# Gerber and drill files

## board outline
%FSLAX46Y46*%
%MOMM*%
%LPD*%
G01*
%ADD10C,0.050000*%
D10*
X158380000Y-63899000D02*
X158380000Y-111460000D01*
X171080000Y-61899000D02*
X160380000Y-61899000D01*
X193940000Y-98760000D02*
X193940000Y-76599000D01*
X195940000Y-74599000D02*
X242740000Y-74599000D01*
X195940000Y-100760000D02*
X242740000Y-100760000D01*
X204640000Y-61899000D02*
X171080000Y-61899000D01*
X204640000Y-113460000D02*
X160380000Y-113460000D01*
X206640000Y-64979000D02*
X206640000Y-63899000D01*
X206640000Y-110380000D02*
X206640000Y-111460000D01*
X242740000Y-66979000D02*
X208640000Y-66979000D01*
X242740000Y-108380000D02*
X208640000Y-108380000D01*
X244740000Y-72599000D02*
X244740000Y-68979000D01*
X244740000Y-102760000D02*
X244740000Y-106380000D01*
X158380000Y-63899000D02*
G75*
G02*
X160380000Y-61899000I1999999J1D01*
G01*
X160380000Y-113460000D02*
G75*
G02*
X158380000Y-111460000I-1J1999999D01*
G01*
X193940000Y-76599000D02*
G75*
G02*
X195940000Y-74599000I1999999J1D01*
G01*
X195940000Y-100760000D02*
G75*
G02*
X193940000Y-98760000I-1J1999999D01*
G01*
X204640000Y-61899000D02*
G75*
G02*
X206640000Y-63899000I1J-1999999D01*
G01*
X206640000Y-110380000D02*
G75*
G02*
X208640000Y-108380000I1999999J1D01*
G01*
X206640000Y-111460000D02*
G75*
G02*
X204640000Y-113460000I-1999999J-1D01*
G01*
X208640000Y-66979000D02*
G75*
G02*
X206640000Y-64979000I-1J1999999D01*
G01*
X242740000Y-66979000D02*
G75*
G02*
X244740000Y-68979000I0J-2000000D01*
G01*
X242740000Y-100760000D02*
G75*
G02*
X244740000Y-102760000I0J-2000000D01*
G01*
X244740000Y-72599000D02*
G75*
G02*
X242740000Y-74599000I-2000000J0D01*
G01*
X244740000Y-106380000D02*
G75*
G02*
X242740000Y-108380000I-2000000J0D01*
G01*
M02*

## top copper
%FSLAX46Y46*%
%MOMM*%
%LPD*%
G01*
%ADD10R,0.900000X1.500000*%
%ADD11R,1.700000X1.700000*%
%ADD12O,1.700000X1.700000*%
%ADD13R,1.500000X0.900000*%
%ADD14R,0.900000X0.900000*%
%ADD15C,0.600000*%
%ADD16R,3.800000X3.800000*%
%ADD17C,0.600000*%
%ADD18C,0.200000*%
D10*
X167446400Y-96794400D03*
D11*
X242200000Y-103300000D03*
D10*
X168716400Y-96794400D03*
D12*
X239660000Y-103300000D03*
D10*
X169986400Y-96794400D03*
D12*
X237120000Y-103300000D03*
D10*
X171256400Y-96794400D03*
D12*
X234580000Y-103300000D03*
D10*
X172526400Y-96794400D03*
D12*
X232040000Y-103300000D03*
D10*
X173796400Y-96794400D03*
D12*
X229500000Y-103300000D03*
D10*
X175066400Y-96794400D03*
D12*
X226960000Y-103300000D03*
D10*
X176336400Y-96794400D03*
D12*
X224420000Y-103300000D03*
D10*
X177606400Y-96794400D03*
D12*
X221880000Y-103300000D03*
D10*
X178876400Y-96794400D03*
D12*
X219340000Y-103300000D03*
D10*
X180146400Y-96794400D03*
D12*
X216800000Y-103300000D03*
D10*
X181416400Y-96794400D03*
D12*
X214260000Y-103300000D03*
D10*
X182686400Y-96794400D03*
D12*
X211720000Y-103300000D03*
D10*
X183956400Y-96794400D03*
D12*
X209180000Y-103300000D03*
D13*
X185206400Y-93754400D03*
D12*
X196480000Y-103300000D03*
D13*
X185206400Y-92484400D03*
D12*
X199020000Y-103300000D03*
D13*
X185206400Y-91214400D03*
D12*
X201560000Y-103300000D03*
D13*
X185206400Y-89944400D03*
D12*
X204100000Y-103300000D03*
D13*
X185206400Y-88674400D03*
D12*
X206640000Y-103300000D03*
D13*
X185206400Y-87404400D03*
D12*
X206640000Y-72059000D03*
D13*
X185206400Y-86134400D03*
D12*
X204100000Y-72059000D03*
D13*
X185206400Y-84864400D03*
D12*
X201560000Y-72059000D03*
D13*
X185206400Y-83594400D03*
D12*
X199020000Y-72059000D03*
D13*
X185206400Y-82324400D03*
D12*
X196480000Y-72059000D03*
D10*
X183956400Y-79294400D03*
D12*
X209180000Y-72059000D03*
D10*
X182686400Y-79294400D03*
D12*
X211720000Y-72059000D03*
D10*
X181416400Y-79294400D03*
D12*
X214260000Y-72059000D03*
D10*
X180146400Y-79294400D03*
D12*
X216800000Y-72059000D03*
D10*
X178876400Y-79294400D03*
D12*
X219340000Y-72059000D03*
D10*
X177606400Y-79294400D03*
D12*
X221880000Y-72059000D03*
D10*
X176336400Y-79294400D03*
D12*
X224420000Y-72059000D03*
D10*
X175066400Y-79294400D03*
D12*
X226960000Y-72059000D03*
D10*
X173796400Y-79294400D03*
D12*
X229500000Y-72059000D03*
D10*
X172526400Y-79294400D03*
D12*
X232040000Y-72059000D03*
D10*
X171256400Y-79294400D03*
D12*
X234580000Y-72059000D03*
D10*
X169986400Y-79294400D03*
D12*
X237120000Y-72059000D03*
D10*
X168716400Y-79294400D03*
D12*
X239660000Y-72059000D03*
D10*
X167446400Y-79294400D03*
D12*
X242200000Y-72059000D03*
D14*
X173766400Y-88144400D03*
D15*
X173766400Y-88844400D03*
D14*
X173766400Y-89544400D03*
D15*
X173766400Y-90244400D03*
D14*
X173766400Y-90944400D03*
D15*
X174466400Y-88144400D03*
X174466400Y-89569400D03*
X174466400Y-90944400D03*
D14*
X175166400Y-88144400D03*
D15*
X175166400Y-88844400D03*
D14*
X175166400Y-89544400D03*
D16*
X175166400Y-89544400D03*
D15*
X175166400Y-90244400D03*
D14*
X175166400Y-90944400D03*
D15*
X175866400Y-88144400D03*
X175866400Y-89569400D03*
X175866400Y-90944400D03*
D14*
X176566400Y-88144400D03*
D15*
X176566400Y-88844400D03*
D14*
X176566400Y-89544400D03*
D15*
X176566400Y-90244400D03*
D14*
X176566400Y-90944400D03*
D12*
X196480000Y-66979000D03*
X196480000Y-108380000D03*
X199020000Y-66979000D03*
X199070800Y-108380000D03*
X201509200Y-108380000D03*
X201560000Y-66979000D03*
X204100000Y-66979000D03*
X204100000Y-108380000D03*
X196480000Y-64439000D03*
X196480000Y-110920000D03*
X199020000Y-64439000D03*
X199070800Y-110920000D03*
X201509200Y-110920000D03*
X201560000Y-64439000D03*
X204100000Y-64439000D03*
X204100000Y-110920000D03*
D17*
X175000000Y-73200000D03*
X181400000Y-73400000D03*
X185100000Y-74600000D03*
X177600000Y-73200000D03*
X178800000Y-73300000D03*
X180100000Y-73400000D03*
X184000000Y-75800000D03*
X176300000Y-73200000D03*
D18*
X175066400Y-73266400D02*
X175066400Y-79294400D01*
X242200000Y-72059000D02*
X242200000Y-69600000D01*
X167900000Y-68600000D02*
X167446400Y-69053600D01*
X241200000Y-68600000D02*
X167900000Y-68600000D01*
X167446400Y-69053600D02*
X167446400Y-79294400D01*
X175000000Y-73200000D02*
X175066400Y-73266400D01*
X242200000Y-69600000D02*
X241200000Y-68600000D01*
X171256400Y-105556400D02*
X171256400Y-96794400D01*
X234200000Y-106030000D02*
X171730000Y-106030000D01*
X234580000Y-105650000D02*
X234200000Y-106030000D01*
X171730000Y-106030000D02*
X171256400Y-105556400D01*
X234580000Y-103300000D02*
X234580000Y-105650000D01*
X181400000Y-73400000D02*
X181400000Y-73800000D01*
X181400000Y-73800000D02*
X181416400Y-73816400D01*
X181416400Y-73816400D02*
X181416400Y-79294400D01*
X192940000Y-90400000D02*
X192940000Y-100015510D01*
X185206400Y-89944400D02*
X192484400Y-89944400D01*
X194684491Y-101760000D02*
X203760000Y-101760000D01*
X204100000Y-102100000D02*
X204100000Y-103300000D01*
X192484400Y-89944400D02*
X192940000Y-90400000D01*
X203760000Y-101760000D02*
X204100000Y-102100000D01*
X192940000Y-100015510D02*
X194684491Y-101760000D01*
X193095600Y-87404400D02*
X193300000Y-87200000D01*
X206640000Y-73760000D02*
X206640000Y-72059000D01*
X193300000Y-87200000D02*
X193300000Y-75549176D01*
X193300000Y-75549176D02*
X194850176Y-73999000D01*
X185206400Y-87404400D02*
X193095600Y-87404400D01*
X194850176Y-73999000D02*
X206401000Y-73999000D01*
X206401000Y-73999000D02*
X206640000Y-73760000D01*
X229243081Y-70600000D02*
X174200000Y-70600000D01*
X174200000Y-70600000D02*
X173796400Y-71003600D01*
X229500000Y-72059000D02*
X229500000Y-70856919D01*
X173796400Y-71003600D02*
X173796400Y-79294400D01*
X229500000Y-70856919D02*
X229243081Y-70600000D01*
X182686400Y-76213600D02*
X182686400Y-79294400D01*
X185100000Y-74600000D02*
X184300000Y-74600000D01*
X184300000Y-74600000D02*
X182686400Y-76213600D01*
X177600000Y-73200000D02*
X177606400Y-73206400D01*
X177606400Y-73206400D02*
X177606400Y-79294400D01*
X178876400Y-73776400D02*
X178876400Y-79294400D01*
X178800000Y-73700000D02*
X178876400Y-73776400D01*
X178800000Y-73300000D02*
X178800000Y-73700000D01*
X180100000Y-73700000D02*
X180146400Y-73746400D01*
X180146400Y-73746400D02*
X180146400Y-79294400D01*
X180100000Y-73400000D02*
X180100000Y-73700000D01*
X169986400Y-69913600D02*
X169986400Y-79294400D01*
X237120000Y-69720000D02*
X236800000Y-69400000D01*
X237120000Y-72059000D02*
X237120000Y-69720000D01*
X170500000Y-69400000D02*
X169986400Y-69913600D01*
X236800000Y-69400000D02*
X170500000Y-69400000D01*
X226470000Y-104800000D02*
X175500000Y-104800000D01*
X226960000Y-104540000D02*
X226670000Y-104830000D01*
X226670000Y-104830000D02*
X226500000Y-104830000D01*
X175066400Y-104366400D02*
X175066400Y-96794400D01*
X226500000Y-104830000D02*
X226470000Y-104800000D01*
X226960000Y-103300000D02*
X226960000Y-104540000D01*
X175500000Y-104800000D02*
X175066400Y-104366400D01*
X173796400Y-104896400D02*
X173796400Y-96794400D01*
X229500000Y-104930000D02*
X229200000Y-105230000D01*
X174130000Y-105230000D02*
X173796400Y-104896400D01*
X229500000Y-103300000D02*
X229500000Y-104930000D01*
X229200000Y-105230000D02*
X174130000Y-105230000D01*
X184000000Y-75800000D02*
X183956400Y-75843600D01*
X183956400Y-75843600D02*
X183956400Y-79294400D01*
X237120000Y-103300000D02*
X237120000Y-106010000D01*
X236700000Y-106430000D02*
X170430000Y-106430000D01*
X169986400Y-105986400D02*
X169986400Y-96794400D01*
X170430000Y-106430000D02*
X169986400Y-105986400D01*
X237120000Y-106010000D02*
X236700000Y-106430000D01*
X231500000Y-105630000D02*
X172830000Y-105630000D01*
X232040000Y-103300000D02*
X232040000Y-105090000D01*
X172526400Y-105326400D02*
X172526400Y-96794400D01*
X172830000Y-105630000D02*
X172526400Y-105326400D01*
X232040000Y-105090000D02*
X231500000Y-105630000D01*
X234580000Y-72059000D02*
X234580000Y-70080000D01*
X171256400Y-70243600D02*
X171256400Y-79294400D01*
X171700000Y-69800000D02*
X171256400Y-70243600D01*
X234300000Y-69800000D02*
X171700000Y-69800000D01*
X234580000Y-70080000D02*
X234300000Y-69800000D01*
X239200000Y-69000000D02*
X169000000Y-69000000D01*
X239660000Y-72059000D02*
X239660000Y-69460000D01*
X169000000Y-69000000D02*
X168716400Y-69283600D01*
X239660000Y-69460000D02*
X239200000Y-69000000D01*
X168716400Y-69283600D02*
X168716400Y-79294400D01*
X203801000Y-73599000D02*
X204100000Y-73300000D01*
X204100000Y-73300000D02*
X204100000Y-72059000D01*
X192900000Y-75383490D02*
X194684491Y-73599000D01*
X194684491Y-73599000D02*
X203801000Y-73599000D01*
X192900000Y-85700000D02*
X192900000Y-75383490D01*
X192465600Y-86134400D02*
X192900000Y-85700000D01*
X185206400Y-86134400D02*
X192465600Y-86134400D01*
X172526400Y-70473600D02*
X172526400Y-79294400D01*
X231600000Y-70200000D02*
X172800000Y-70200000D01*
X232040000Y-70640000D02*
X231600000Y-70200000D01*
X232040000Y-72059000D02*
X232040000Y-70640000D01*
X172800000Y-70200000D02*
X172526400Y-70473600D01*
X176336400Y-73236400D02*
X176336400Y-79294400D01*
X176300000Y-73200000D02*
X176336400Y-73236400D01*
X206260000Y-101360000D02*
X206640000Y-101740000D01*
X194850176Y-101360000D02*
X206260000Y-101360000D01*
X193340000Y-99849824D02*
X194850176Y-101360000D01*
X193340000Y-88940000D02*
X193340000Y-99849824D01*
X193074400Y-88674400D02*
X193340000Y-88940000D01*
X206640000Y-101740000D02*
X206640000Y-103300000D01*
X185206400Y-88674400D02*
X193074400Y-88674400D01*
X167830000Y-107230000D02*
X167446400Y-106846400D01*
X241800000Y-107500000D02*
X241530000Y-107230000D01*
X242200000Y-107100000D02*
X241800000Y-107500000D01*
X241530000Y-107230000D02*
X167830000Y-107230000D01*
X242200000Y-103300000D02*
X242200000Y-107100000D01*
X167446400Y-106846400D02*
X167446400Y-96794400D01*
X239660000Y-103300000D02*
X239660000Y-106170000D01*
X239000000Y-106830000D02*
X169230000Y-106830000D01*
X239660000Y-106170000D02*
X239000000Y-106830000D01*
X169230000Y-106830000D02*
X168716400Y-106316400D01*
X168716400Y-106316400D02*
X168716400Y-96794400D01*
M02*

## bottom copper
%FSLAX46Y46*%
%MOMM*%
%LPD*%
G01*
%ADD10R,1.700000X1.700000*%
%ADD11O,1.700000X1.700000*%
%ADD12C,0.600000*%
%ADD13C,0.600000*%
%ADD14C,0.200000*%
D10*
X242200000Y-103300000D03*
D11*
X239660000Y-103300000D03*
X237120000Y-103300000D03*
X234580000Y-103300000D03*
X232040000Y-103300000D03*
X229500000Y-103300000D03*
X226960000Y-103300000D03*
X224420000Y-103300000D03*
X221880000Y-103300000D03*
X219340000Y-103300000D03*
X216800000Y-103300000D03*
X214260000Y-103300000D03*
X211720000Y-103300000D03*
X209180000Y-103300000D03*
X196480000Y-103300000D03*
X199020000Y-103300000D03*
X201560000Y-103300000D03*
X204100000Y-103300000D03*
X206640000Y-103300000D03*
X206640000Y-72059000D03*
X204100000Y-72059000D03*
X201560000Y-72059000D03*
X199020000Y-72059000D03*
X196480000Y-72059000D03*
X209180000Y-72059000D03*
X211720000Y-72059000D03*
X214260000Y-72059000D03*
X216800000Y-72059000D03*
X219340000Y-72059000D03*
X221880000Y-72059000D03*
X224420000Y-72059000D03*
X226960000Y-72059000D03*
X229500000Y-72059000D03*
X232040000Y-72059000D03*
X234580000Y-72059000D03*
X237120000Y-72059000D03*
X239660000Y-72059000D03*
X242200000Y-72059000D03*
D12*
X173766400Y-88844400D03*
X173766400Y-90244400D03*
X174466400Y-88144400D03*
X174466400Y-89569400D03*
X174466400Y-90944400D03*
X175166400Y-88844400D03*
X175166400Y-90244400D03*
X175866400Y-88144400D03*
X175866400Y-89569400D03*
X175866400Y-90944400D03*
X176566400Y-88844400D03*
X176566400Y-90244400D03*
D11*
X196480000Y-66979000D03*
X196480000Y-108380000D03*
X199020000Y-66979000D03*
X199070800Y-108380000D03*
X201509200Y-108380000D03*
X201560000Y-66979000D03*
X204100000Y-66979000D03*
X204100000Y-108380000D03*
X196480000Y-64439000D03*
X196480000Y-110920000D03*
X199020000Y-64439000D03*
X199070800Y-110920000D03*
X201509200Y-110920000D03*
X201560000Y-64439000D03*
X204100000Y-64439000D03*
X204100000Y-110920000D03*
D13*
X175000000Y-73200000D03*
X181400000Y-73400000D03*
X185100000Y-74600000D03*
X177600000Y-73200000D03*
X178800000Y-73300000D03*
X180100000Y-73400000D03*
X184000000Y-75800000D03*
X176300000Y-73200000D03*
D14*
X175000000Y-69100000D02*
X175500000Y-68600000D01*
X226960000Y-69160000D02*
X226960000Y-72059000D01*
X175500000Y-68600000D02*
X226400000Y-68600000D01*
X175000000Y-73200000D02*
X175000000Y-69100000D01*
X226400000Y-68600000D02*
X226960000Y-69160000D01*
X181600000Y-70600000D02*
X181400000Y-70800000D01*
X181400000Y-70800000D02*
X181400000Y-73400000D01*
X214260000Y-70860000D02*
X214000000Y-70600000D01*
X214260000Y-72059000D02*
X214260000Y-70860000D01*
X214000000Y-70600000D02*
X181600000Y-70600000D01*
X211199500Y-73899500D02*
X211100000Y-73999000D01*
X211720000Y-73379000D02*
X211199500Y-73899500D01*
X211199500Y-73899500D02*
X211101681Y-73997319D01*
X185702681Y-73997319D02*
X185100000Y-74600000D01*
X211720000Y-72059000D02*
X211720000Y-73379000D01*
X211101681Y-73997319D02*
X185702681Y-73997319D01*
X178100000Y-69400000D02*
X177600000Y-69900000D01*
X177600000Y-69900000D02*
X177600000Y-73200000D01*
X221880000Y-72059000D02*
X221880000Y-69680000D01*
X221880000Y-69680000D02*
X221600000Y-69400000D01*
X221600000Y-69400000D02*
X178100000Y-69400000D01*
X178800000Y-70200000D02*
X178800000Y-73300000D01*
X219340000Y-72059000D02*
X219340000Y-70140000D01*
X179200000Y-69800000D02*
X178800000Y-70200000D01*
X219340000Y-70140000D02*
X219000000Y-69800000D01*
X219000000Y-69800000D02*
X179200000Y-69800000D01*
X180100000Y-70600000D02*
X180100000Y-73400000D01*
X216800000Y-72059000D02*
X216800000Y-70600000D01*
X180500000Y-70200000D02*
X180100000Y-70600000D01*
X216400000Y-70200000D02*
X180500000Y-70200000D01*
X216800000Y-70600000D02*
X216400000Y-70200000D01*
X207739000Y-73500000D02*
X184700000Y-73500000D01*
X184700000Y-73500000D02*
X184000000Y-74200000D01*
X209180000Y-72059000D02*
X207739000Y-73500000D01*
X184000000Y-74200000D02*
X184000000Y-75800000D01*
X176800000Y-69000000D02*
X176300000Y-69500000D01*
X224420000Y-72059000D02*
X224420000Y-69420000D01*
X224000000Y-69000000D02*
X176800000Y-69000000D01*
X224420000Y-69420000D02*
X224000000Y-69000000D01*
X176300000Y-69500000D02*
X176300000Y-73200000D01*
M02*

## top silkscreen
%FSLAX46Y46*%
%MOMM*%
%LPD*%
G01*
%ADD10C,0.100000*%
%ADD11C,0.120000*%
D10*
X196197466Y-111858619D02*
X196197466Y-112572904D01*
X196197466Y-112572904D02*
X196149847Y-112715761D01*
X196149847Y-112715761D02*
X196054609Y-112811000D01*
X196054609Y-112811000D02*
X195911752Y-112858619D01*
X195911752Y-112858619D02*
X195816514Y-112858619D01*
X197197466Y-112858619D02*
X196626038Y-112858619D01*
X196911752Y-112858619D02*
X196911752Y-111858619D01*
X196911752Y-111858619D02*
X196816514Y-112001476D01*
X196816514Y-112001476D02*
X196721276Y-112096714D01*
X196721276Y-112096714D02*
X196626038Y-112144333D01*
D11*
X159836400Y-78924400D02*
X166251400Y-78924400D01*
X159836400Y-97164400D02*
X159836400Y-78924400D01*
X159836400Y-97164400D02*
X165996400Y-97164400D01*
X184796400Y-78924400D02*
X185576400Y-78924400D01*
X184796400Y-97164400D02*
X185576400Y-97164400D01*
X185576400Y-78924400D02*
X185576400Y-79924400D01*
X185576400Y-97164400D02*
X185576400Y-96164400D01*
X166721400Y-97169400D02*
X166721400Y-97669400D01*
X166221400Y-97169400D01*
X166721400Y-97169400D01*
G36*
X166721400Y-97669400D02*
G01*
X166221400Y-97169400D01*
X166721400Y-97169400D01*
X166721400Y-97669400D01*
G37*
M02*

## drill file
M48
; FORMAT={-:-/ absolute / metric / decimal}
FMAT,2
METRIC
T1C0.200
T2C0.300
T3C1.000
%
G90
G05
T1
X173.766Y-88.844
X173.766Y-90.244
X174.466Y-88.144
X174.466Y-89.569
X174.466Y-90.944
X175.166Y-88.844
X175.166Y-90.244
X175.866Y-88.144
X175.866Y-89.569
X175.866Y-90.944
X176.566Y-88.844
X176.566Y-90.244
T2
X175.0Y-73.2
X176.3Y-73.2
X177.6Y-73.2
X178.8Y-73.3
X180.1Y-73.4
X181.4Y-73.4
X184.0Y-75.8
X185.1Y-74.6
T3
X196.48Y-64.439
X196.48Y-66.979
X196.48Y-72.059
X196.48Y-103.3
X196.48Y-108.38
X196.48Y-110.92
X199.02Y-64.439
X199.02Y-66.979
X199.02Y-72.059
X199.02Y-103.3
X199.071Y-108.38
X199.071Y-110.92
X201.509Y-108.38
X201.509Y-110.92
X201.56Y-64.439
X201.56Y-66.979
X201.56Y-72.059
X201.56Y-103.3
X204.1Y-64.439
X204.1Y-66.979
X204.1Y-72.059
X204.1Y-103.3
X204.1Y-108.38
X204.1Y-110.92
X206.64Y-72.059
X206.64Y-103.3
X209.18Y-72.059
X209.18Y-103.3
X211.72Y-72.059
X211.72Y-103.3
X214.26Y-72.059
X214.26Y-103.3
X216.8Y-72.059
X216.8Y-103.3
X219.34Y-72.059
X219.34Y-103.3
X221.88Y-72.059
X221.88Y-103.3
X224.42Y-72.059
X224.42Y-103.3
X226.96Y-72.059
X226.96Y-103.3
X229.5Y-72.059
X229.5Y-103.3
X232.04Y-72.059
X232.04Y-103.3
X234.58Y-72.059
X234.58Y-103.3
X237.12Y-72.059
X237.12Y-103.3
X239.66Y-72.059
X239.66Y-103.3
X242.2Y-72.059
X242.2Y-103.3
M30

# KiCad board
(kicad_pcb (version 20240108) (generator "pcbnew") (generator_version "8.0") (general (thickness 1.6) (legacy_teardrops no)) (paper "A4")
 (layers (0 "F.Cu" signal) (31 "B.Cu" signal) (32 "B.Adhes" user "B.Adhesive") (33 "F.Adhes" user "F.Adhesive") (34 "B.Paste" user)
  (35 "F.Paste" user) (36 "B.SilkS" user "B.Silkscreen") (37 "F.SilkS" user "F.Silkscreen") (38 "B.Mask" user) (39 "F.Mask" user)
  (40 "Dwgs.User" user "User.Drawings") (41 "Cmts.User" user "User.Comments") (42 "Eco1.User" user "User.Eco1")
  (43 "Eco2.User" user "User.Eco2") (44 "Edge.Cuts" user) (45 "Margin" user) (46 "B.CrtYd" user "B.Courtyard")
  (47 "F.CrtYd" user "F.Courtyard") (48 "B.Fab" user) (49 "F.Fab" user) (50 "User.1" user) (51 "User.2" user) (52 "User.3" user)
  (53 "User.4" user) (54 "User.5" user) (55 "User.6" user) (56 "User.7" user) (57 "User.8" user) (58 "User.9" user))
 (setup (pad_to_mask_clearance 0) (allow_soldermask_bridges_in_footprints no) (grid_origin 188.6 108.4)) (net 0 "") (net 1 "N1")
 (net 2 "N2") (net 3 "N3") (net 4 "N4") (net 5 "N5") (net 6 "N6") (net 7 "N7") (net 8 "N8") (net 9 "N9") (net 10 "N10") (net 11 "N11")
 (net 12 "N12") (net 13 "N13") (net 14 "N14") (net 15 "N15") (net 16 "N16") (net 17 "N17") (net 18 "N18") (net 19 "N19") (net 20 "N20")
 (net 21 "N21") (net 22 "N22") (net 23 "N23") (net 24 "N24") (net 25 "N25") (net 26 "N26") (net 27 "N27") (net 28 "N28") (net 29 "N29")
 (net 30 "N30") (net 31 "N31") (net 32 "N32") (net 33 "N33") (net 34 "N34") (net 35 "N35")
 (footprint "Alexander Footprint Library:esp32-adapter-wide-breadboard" (layer "F.Cu") (at 211.72 108.38)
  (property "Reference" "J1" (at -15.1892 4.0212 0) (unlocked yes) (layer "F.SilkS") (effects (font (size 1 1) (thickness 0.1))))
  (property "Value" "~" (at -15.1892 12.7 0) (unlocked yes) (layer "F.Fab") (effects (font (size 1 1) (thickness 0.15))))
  (fp_line (start -51.8836 -29.4556) (end -45.4686 -29.4556) (stroke (width 0.12) (type solid)) (layer "F.SilkS"))
  (fp_line (start -51.8836 -11.2156) (end -51.8836 -29.4556) (stroke (width 0.12) (type solid)) (layer "F.SilkS"))
  (fp_line (start -51.8836 -11.2156) (end -45.7236 -11.2156) (stroke (width 0.12) (type solid)) (layer "F.SilkS"))
  (fp_line (start -26.9236 -29.4556) (end -26.1436 -29.4556) (stroke (width 0.12) (type solid)) (layer "F.SilkS"))
  (fp_line (start -26.9236 -11.2156) (end -26.1436 -11.2156) (stroke (width 0.12) (type solid)) (layer "F.SilkS"))
  (fp_line (start -26.1436 -29.4556) (end -26.1436 -28.4556) (stroke (width 0.12) (type solid)) (layer "F.SilkS"))
  (fp_line (start -26.1436 -11.2156) (end -26.1436 -12.2156) (stroke (width 0.12) (type solid)) (layer "F.SilkS"))
  (fp_poly
   (pts (xy -44.9986 -11.2106) (xy -44.9986 -10.7106) (xy -45.4986 -11.2106) (xy -44.9986 -11.2106)) (stroke (width 0.12) (type solid))
   (fill solid) (layer "F.SilkS"))
  (fp_line (start -53.34 -44.481) (end -53.34 3.08) (stroke (width 0.05) (type default)) (layer "Edge.Cuts"))
  (fp_line (start -40.64 -46.481) (end -51.34 -46.481) (stroke (width 0.05) (type default)) (layer "Edge.Cuts"))
  (fp_line (start -17.78 -9.62) (end -17.78 -31.781) (stroke (width 0.05) (type default)) (layer "Edge.Cuts"))
  (fp_line (start -15.78 -33.781) (end 31.02 -33.781) (stroke (width 0.05) (type default)) (layer "Edge.Cuts"))
  (fp_line (start -15.78 -7.62) (end 31.02 -7.62) (stroke (width 0.05) (type default)) (layer "Edge.Cuts"))
  (fp_line (start -7.08 -46.481) (end -40.64 -46.481) (stroke (width 0.05) (type default)) (layer "Edge.Cuts"))
  (fp_line (start -7.08 5.08) (end -51.34 5.08) (stroke (width 0.05) (type default)) (layer "Edge.Cuts"))
  (fp_line (start -5.08 -43.401) (end -5.08 -44.481) (stroke (width 0.05) (type default)) (layer "Edge.Cuts"))
  (fp_line (start -5.08 2) (end -5.08 3.08) (stroke (width 0.05) (type default)) (layer "Edge.Cuts"))
  (fp_line (start 31.02 -41.401) (end -3.08 -41.401) (stroke (width 0.05) (type default)) (layer "Edge.Cuts"))
  (fp_line (start 31.02 0) (end -3.08 0) (stroke (width 0.05) (type default)) (layer "Edge.Cuts"))
  (fp_line (start 33.02 -35.781) (end 33.02 -39.401) (stroke (width 0.05) (type default)) (layer "Edge.Cuts"))
  (fp_line (start 33.02 -5.62) (end 33.02 -2) (stroke (width 0.05) (type default)) (layer "Edge.Cuts"))
  (fp_arc (start -53.34 -44.481) (mid -52.754214 -45.895214) (end -51.34 -46.481) (stroke (width 0.05) (type default)) (layer "Edge.Cuts"))
  (fp_arc (start -51.34 5.08) (mid -52.754214 4.494214) (end -53.34 3.08) (stroke (width 0.05) (type default)) (layer "Edge.Cuts"))
  (fp_arc (start -17.78 -31.781) (mid -17.194214 -33.195214) (end -15.78 -33.781) (stroke (width 0.05) (type default)) (layer "Edge.Cuts"))
  (fp_arc (start -15.78 -7.62) (mid -17.194214 -8.205786) (end -17.78 -9.62) (stroke (width 0.05) (type default)) (layer "Edge.Cuts"))
  (fp_arc (start -7.08 -46.481) (mid -5.665786 -45.895214) (end -5.08 -44.481) (stroke (width 0.05) (type default)) (layer "Edge.Cuts"))
  (fp_arc (start -5.08 2) (mid -4.494214 0.585786) (end -3.08 0) (stroke (width 0.05) (type default)) (layer "Edge.Cuts"))
  (fp_arc (start -5.08 3.08) (mid -5.665786 4.494214) (end -7.08 5.08) (stroke (width 0.05) (type default)) (layer "Edge.Cuts"))
  (fp_arc (start -3.08 -41.401) (mid -4.494214 -41.986786) (end -5.08 -43.401) (stroke (width 0.05) (type default)) (layer "Edge.Cuts"))
  (fp_arc (start 31.02 -41.401) (mid 32.434214 -40.815214) (end 33.02 -39.401) (stroke (width 0.05) (type default)) (layer "Edge.Cuts"))
  (fp_arc (start 31.02 -7.62) (mid 32.434214 -7.034214) (end 33.02 -5.62) (stroke (width 0.05) (type default)) (layer "Edge.Cuts"))
  (fp_arc (start 33.02 -35.781) (mid 32.434214 -34.366786) (end 31.02 -33.781) (stroke (width 0.05) (type default)) (layer "Edge.Cuts"))
  (fp_arc (start 33.02 -2) (mid 32.434214 -0.585786) (end 31.02 0) (stroke (width 0.05) (type default)) (layer "Edge.Cuts"))
  (pad "1" smd rect (at -44.2736 -11.5856 90) (size 1.5 0.9) (layers "F.Cu" "F.Paste" "F.Mask") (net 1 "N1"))
  (pad "1" thru_hole rect (at 30.48 -5.08 270) (size 1.7 1.7) (drill 1) (layers "*.Cu" "*.Mask") (remove_unused_layers no) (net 1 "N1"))
  (pad "2" smd rect (at -43.0036 -11.5856 90) (size 1.5 0.9) (layers "F.Cu" "F.Paste" "F.Mask") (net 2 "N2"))
  (pad "2" thru_hole oval (at 27.94 -5.08) (size 1.7 1.7) (drill 1) (layers "*.Cu" "*.Mask") (remove_unused_layers no) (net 2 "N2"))
  (pad "3" smd rect (at -41.7336 -11.5856 90) (size 1.5 0.9) (layers "F.Cu" "F.Paste" "F.Mask") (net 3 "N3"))
  (pad "3" thru_hole oval (at 25.4 -5.08) (size 1.7 1.7) (drill 1) (layers "*.Cu" "*.Mask") (remove_unused_layers no) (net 3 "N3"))
  (pad "4" smd rect (at -40.4636 -11.5856 90) (size 1.5 0.9) (layers "F.Cu" "F.Paste" "F.Mask") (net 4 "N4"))
  (pad "4" thru_hole oval (at 22.86 -5.08) (size 1.7 1.7) (drill 1) (layers "*.Cu" "*.Mask") (remove_unused_layers no) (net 4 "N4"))
  (pad "5" smd rect (at -39.1936 -11.5856 90) (size 1.5 0.9) (layers "F.Cu" "F.Paste" "F.Mask") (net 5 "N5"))
  (pad "5" thru_hole oval (at 20.32 -5.08) (size 1.7 1.7) (drill 1) (layers "*.Cu" "*.Mask") (remove_unused_layers no) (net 5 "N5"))
  (pad "6" smd rect (at -37.9236 -11.5856 90) (size 1.5 0.9) (layers "F.Cu" "F.Paste" "F.Mask") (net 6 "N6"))
  (pad "6" thru_hole oval (at 17.78 -5.08) (size 1.7 1.7) (drill 1) (layers "*.Cu" "*.Mask") (remove_unused_layers no) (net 6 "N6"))
  (pad "7" smd rect (at -36.6536 -11.5856 90) (size 1.5 0.9) (layers "F.Cu" "F.Paste" "F.Mask") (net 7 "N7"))
  (pad "7" thru_hole oval (at 15.24 -5.08) (size 1.7 1.7) (drill 1) (layers "*.Cu" "*.Mask") (remove_unused_layers no) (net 7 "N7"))
  (pad "8" smd rect (at -35.3836 -11.5856 90) (size 1.5 0.9) (layers "F.Cu" "F.Paste" "F.Mask") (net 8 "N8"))
  (pad "8" thru_hole oval (at 12.7 -5.08) (size 1.7 1.7) (drill 1) (layers "*.Cu" "*.Mask") (remove_unused_layers no) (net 8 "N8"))
  (pad "9" smd rect (at -34.1136 -11.5856 90) (size 1.5 0.9) (layers "F.Cu" "F.Paste" "F.Mask") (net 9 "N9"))
  (pad "9" thru_hole oval (at 10.16 -5.08) (size 1.7 1.7) (drill 1) (layers "*.Cu" "*.Mask") (remove_unused_layers no) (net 9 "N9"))
  (pad "10" smd rect (at -32.8436 -11.5856 90) (size 1.5 0.9) (layers "F.Cu" "F.Paste" "F.Mask") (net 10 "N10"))
  (pad "10" thru_hole oval (at 7.62 -5.08) (size 1.7 1.7) (drill 1) (layers "*.Cu" "*.Mask") (remove_unused_layers no) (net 10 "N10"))
  (pad "11" smd rect (at -31.5736 -11.5856 90) (size 1.5 0.9) (layers "F.Cu" "F.Paste" "F.Mask") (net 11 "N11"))
  (pad "11" thru_hole oval (at 5.08 -5.08) (size 1.7 1.7) (drill 1) (layers "*.Cu" "*.Mask") (remove_unused_layers no) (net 11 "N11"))
  (pad "12" smd rect (at -30.3036 -11.5856 90) (size 1.5 0.9) (layers "F.Cu" "F.Paste" "F.Mask") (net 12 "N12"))
  (pad "12" thru_hole oval (at 2.54 -5.08) (size 1.7 1.7) (drill 1) (layers "*.Cu" "*.Mask") (remove_unused_layers no) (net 12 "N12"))
  (pad "13" smd rect (at -29.0336 -11.5856 90) (size 1.5 0.9) (layers "F.Cu" "F.Paste" "F.Mask") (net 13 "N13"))
  (pad "13" thru_hole oval (at 0 -5.08) (size 1.7 1.7) (drill 1) (layers "*.Cu" "*.Mask") (remove_unused_layers no) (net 13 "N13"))
  (pad "14" smd rect (at -27.7636 -11.5856 90) (size 1.5 0.9) (layers "F.Cu" "F.Paste" "F.Mask") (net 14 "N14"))
  (pad "14" thru_hole oval (at -2.54 -5.08) (size 1.7 1.7) (drill 1) (layers "*.Cu" "*.Mask") (remove_unused_layers no) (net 14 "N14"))
  (pad "15" smd rect (at -26.5136 -14.6256 180) (size 1.5 0.9) (layers "F.Cu" "F.Paste" "F.Mask"))
  (pad "15" thru_hole oval (at -15.24 -5.08) (size 1.7 1.7) (drill 1) (layers "*.Cu" "*.Mask") (remove_unused_layers no))
  (pad "16" smd rect (at -26.5136 -15.8956 180) (size 1.5 0.9) (layers "F.Cu" "F.Paste" "F.Mask") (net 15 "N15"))
  (pad "16" thru_hole oval (at -12.7 -5.08) (size 1.7 1.7) (drill 1) (layers "*.Cu" "*.Mask") (remove_unused_layers no) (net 15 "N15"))
  (pad "17" smd rect (at -26.5136 -17.1656 180) (size 1.5 0.9) (layers "F.Cu" "F.Paste" "F.Mask") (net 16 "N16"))
  (pad "17" thru_hole oval (at -10.16 -5.08) (size 1.7 1.7) (drill 1) (layers "*.Cu" "*.Mask") (remove_unused_layers no) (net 16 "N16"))
  (pad "18" smd rect (at -26.5136 -18.4356 180) (size 1.5 0.9) (layers "F.Cu" "F.Paste" "F.Mask") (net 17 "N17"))
  (pad "18" thru_hole oval (at -7.62 -5.08) (size 1.7 1.7) (drill 1) (layers "*.Cu" "*.Mask") (remove_unused_layers no) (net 17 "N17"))
  (pad "19" smd rect (at -26.5136 -19.7056 180) (size 1.5 0.9) (layers "F.Cu" "F.Paste" "F.Mask") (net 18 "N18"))
  (pad "19" thru_hole oval (at -5.08 -5.08) (size 1.7 1.7) (drill 1) (layers "*.Cu" "*.Mask") (remove_unused_layers no) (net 18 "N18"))
  (pad "20" smd rect (at -26.5136 -20.9756 180) (size 1.5 0.9) (layers "F.Cu" "F.Paste" "F.Mask") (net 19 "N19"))
  (pad "20" thru_hole oval (at -5.08 -36.321) (size 1.7 1.7) (drill 1) (layers "*.Cu" "*.Mask") (remove_unused_layers no) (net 19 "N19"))
  (pad "21" smd rect (at -26.5136 -22.2456 180) (size 1.5 0.9) (layers "F.Cu" "F.Paste" "F.Mask") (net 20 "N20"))
  (pad "21" thru_hole oval (at -7.62 -36.321) (size 1.7 1.7) (drill 1) (layers "*.Cu" "*.Mask") (remove_unused_layers no) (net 20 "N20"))
  (pad "22" smd rect (at -26.5136 -23.5156 180) (size 1.5 0.9) (layers "F.Cu" "F.Paste" "F.Mask") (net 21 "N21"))
  (pad "22" thru_hole oval (at -10.16 -36.321) (size 1.7 1.7) (drill 1) (layers "*.Cu" "*.Mask") (remove_unused_layers no) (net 21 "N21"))
  (pad "23" smd rect (at -26.5136 -24.7856 180) (size 1.5 0.9) (layers "F.Cu" "F.Paste" "F.Mask") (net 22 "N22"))
  (pad "23" thru_hole oval (at -12.7 -36.321) (size 1.7 1.7) (drill 1) (layers "*.Cu" "*.Mask") (remove_unused_layers no) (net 22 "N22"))
  (pad "24" smd rect (at -26.5136 -26.0556 180) (size 1.5 0.9) (layers "F.Cu" "F.Paste" "F.Mask") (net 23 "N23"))
  (pad "24" thru_hole oval (at -15.24 -36.321) (size 1.7 1.7) (drill 1) (layers "*.Cu" "*.Mask") (remove_unused_layers no) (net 23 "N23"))
  (pad "25" smd rect (at -27.7636 -29.0856 90) (size 1.5 0.9) (layers "F.Cu" "F.Paste" "F.Mask") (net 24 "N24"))
  (pad "25" thru_hole oval (at -2.54 -36.321) (size 1.7 1.7) (drill 1) (layers "*.Cu" "*.Mask") (remove_unused_layers no) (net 24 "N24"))
  (pad "26" smd rect (at -29.0336 -29.0856 90) (size 1.5 0.9) (layers "F.Cu" "F.Paste" "F.Mask") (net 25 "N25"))
  (pad "26" thru_hole oval (at 0 -36.321) (size 1.7 1.7) (drill 1) (layers "*.Cu" "*.Mask") (remove_unused_layers no) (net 25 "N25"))
  (pad "27" smd rect (at -30.3036 -29.0856 90) (size 1.5 0.9) (layers "F.Cu" "F.Paste" "F.Mask") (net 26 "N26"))
  (pad "27" thru_hole oval (at 2.54 -36.321) (size 1.7 1.7) (drill 1) (layers "*.Cu" "*.Mask") (remove_unused_layers no) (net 26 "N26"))
  (pad "28" smd rect (at -31.5736 -29.0856 90) (size 1.5 0.9) (layers "F.Cu" "F.Paste" "F.Mask") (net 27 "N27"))
  (pad "28" thru_hole oval (at 5.08 -36.321) (size 1.7 1.7) (drill 1) (layers "*.Cu" "*.Mask") (remove_unused_layers no) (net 27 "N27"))
  (pad "29" smd rect (at -32.8436 -29.0856 90) (size 1.5 0.9) (layers "F.Cu" "F.Paste" "F.Mask") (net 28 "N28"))
  (pad "29" thru_hole oval (at 7.62 -36.321) (size 1.7 1.7) (drill 1) (layers "*.Cu" "*.Mask") (remove_unused_layers no) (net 28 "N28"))
  (pad "30" smd rect (at -34.1136 -29.0856 90) (size 1.5 0.9) (layers "F.Cu" "F.Paste" "F.Mask") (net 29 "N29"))
  (pad "30" thru_hole oval (at 10.16 -36.321) (size 1.7 1.7) (drill 1) (layers "*.Cu" "*.Mask") (remove_unused_layers no) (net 29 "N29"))
  (pad "31" smd rect (at -35.3836 -29.0856 90) (size 1.5 0.9) (layers "F.Cu" "F.Paste" "F.Mask") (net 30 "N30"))
  (pad "31" thru_hole oval (at 12.7 -36.321) (size 1.7 1.7) (drill 1) (layers "*.Cu" "*.Mask") (remove_unused_layers no) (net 30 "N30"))
  (pad "32" smd rect (at -36.6536 -29.0856 90) (size 1.5 0.9) (layers "F.Cu" "F.Paste" "F.Mask"))
  (pad "32" thru_hole oval (at 15.24 -36.321) (size 1.7 1.7) (drill 1) (layers "*.Cu" "*.Mask") (remove_unused_layers no))
  (pad "33" smd rect (at -37.9236 -29.0856 90) (size 1.5 0.9) (layers "F.Cu" "F.Paste" "F.Mask") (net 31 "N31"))
  (pad "33" thru_hole oval (at 17.78 -36.321) (size 1.7 1.7) (drill 1) (layers "*.Cu" "*.Mask") (remove_unused_layers no) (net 31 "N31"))
  (pad "34" smd rect (at -39.1936 -29.0856 90) (size 1.5 0.9) (layers "F.Cu" "F.Paste" "F.Mask") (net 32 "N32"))
  (pad "34" thru_hole oval (at 20.32 -36.321) (size 1.7 1.7) (drill 1) (layers "*.Cu" "*.Mask") (remove_unused_layers no) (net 32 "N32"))
  (pad "35" smd rect (at -40.4636 -29.0856 90) (size 1.5 0.9) (layers "F.Cu" "F.Paste" "F.Mask") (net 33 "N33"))
  (pad "35" thru_hole oval (at 22.86 -36.321) (size 1.7 1.7) (drill 1) (layers "*.Cu" "*.Mask") (remove_unused_layers no) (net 33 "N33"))
  (pad "36" smd rect (at -41.7336 -29.0856 90) (size 1.5 0.9) (layers "F.Cu" "F.Paste" "F.Mask") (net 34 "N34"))
  (pad "36" thru_hole oval (at 25.4 -36.321) (size 1.7 1.7) (drill 1) (layers "*.Cu" "*.Mask") (remove_unused_layers no) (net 34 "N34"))
  (pad "37" smd rect (at -43.0036 -29.0856 90) (size 1.5 0.9) (layers "F.Cu" "F.Paste" "F.Mask") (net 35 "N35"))
  (pad "37" thru_hole oval (at 27.94 -36.321) (size 1.7 1.7) (drill 1) (layers "*.Cu" "*.Mask") (remove_unused_layers no) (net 35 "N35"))
  (pad "38" smd rect (at -44.2736 -29.0856 90) (size 1.5 0.9) (layers "F.Cu" "F.Paste" "F.Mask"))
  (pad "38" thru_hole oval (at 30.48 -36.321) (size 1.7 1.7) (drill 1) (layers "*.Cu" "*.Mask") (remove_unused_layers no))
  (pad "39" smd rect (at -37.9536 -20.2356 90) (size 0.9 0.9) (layers "F.Cu" "F.Paste"))
  (pad "39" thru_hole circle (at -37.9536 -19.5356 90) (size 0.6 0.6) (drill 0.2) (layers "*.Cu" "F.Mask") (remove_unused_layers no))
  (pad "39" smd rect (at -37.9536 -18.8356 90) (size 0.9 0.9) (layers "F.Cu" "F.Paste"))
  (pad "39" thru_hole circle (at -37.9536 -18.1356 90) (size 0.6 0.6) (drill 0.2) (layers "*.Cu" "F.Mask") (remove_unused_layers no))
  (pad "39" smd rect (at -37.9536 -17.4356 90) (size 0.9 0.9) (layers "F.Cu" "F.Paste"))
  (pad "39" thru_hole circle (at -37.2536 -20.2356 90) (size 0.6 0.6) (drill 0.2) (layers "*.Cu" "F.Mask") (remove_unused_layers no))
  (pad "39" thru_hole circle (at -37.2536 -18.8106 90) (size 0.6 0.6) (drill 0.2) (layers "*.Cu" "F.Mask") (remove_unused_layers no))
  (pad "39" thru_hole circle (at -37.2536 -17.4356 90) (size 0.6 0.6) (drill 0.2) (layers "*.Cu" "F.Mask") (remove_unused_layers no))
  (pad "39" smd rect (at -36.5536 -20.2356 90) (size 0.9 0.9) (layers "F.Cu" "F.Paste"))
  (pad "39" thru_hole circle (at -36.5536 -19.5356 90) (size 0.6 0.6) (drill 0.2) (layers "*.Cu" "F.Mask") (remove_unused_layers no))
  (pad "39" smd rect (at -36.5536 -18.8356 90) (size 0.9 0.9) (layers "F.Cu" "F.Paste"))
  (pad "39" smd rect (at -36.5536 -18.8356 90) (size 3.8 3.8) (layers "F.Cu" "F.Mask"))
  (pad "39" thru_hole circle (at -36.5536 -18.1356 90) (size 0.6 0.6) (drill 0.2) (layers "*.Cu" "F.Mask") (remove_unused_layers no))
  (pad "39" smd rect (at -36.5536 -17.4356 90) (size 0.9 0.9) (layers "F.Cu" "F.Paste"))
  (pad "39" thru_hole circle (at -35.8536 -20.2356 90) (size 0.6 0.6) (drill 0.2) (layers "*.Cu" "F.Mask") (remove_unused_layers no))
  (pad "39" thru_hole circle (at -35.8536 -18.8106 90) (size 0.6 0.6) (drill 0.2) (layers "*.Cu" "F.Mask") (remove_unused_layers no))
  (pad "39" thru_hole circle (at -35.8536 -17.4356 90) (size 0.6 0.6) (drill 0.2) (layers "*.Cu" "F.Mask") (remove_unused_layers no))
  (pad "39" smd rect (at -35.1536 -20.2356 90) (size 0.9 0.9) (layers "F.Cu" "F.Paste"))
  (pad "39" thru_hole circle (at -35.1536 -19.5356 90) (size 0.6 0.6) (drill 0.2) (layers "*.Cu" "F.Mask") (remove_unused_layers no))
  (pad "39" smd rect (at -35.1536 -18.8356 90) (size 0.9 0.9) (layers "F.Cu" "F.Paste"))
  (pad "39" thru_hole circle (at -35.1536 -18.1356 90) (size 0.6 0.6) (drill 0.2) (layers "*.Cu" "F.Mask") (remove_unused_layers no))
  (pad "39" smd rect (at -35.1536 -17.4356 90) (size 0.9 0.9) (layers "F.Cu" "F.Paste"))
  (pad "GND" thru_hole oval (at -15.24 -41.401) (size 1.7 1.7) (drill 1) (layers "*.Cu" "*.Mask") (remove_unused_layers no))
  (pad "GND" thru_hole oval (at -15.24 0) (size 1.7 1.7) (drill 1) (layers "*.Cu" "*.Mask") (remove_unused_layers no))
  (pad "GND" thru_hole oval (at -12.7 -41.401) (size 1.7 1.7) (drill 1) (layers "*.Cu" "*.Mask") (remove_unused_layers no))
  (pad "GND" thru_hole oval (at -12.6492 0) (size 1.7 1.7) (drill 1) (layers "*.Cu" "*.Mask") (remove_unused_layers no))
  (pad "GND" thru_hole oval (at -10.2108 0) (size 1.7 1.7) (drill 1) (layers "*.Cu" "*.Mask") (remove_unused_layers no))
  (pad "GND" thru_hole oval (at -10.16 -41.401) (size 1.7 1.7) (drill 1) (layers "*.Cu" "*.Mask") (remove_unused_layers no))
  (pad "GND" thru_hole oval (at -7.62 -41.401) (size 1.7 1.7) (drill 1) (layers "*.Cu" "*.Mask") (remove_unused_layers no))
  (pad "GND" thru_hole oval (at -7.62 0) (size 1.7 1.7) (drill 1) (layers "*.Cu" "*.Mask") (remove_unused_layers no))
  (pad "VCC" thru_hole oval (at -15.24 -43.941) (size 1.7 1.7) (drill 1) (layers "*.Cu" "*.Mask") (remove_unused_layers no))
  (pad "VCC" thru_hole oval (at -15.24 2.54) (size 1.7 1.7) (drill 1) (layers "*.Cu" "*.Mask") (remove_unused_layers no))
  (pad "VCC" thru_hole oval (at -12.7 -43.941) (size 1.7 1.7) (drill 1) (layers "*.Cu" "*.Mask") (remove_unused_layers no))
  (pad "VCC" thru_hole oval (at -12.6492 2.54) (size 1.7 1.7) (drill 1) (layers "*.Cu" "*.Mask") (remove_unused_layers no))
  (pad "VCC" thru_hole oval (at -10.2108 2.54) (size 1.7 1.7) (drill 1) (layers "*.Cu" "*.Mask") (remove_unused_layers no))
  (pad "VCC" thru_hole oval (at -10.16 -43.941) (size 1.7 1.7) (drill 1) (layers "*.Cu" "*.Mask") (remove_unused_layers no))
  (pad "VCC" thru_hole oval (at -7.62 -43.941) (size 1.7 1.7) (drill 1) (layers "*.Cu" "*.Mask") (remove_unused_layers no))
  (pad "VCC" thru_hole oval (at -7.62 2.54) (size 1.7 1.7) (drill 1) (layers "*.Cu" "*.Mask") (remove_unused_layers no)))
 (segment (start 175.0664 73.2664) (end 175.0664 79.2944) (width 0.2) (layer "F.Cu") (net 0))
 (segment (start 242.2 72.059) (end 242.2 69.6) (width 0.2) (layer "F.Cu") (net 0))
 (segment (start 167.9 68.6) (end 167.4464 69.0536) (width 0.2) (layer "F.Cu") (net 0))
 (segment (start 241.2 68.6) (end 167.9 68.6) (width 0.2) (layer "F.Cu") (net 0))
 (segment (start 167.4464 69.0536) (end 167.4464 79.2944) (width 0.2) (layer "F.Cu") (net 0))
 (segment (start 175 73.2) (end 175.0664 73.2664) (width 0.2) (layer "F.Cu") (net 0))
 (segment (start 242.2 69.6) (end 241.2 68.6) (width 0.2) (layer "F.Cu") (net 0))
 (via (at 175 73.2) (size 0.6) (drill 0.3) (layers "F.Cu" "B.Cu") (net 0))
 (segment (start 175 69.1) (end 175.5 68.6) (width 0.2) (layer "B.Cu") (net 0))
 (segment (start 226.96 69.16) (end 226.96 72.059) (width 0.2) (layer "B.Cu") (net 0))
 (segment (start 175.5 68.6) (end 226.4 68.6) (width 0.2) (layer "B.Cu") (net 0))
 (segment (start 175 73.2) (end 175 69.1) (width 0.2) (layer "B.Cu") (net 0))
 (segment (start 226.4 68.6) (end 226.96 69.16) (width 0.2) (layer "B.Cu") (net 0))
 (segment (start 171.2564 105.5564) (end 171.2564 96.7944) (width 0.2) (layer "F.Cu") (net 4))
 (segment (start 234.2 106.03) (end 171.73 106.03) (width 0.2) (layer "F.Cu") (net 4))
 (segment (start 234.58 105.65) (end 234.2 106.03) (width 0.2) (layer "F.Cu") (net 4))
 (segment (start 171.73 106.03) (end 171.2564 105.5564) (width 0.2) (layer "F.Cu") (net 4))
 (segment (start 234.58 103.3) (end 234.58 105.65) (width 0.2) (layer "F.Cu") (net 4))
 (segment (start 181.4 73.4) (end 181.4 73.8) (width 0.2) (layer "F.Cu") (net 26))
 (segment (start 181.4 73.8) (end 181.4164 73.8164) (width 0.2) (layer "F.Cu") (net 26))
 (segment (start 181.4164 73.8164) (end 181.4164 79.2944) (width 0.2) (layer "F.Cu") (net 26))
 (via (at 181.4 73.4) (size 0.6) (drill 0.3) (layers "F.Cu" "B.Cu") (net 26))
 (segment (start 181.6 70.6) (end 181.4 70.8) (width 0.2) (layer "B.Cu") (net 26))
 (segment (start 181.4 70.8) (end 181.4 73.4) (width 0.2) (layer "B.Cu") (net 26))
 (segment (start 214.26 70.86) (end 214 70.6) (width 0.2) (layer "B.Cu") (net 26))
 (segment (start 214.26 72.059) (end 214.26 70.86) (width 0.2) (layer "B.Cu") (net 26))
 (segment (start 214 70.6) (end 181.6 70.6) (width 0.2) (layer "B.Cu") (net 26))
 (segment (start 192.94 90.4) (end 192.94 100.01551) (width 0.2) (layer "F.Cu") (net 17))
 (segment (start 185.2064 89.9444) (end 192.4844 89.9444) (width 0.2) (layer "F.Cu") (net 17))
 (segment (start 194.684491 101.76) (end 203.76 101.76) (width 0.2) (layer "F.Cu") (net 17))
 (segment (start 204.1 102.1) (end 204.1 103.3) (width 0.2) (layer "F.Cu") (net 17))
 (segment (start 192.4844 89.9444) (end 192.94 90.4) (width 0.2) (layer "F.Cu") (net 17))
 (segment (start 203.76 101.76) (end 204.1 102.1) (width 0.2) (layer "F.Cu") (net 17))
 (segment (start 192.94 100.01551) (end 194.684491 101.76) (width 0.2) (layer "F.Cu") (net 17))
 (segment (start 193.0956 87.4044) (end 193.3 87.2) (width 0.2) (layer "F.Cu") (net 19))
 (segment (start 206.64 73.76) (end 206.64 72.059) (width 0.2) (layer "F.Cu") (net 19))
 (segment (start 193.3 87.2) (end 193.3 75.549176) (width 0.2) (layer "F.Cu") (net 19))
 (segment (start 193.3 75.549176) (end 194.850176 73.999) (width 0.2) (layer "F.Cu") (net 19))
 (segment (start 185.2064 87.4044) (end 193.0956 87.4044) (width 0.2) (layer "F.Cu") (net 19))
 (segment (start 194.850176 73.999) (end 206.401 73.999) (width 0.2) (layer "F.Cu") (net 19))
 (segment (start 206.401 73.999) (end 206.64 73.76) (width 0.2) (layer "F.Cu") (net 19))
 (segment (start 229.243081 70.6) (end 174.2 70.6) (width 0.2) (layer "F.Cu") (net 31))
 (segment (start 174.2 70.6) (end 173.7964 71.0036) (width 0.2) (layer "F.Cu") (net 31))
 (segment (start 229.5 72.059) (end 229.5 70.856919) (width 0.2) (layer "F.Cu") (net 31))
 (segment (start 173.7964 71.0036) (end 173.7964 79.2944) (width 0.2) (layer "F.Cu") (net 31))
 (segment (start 229.5 70.856919) (end 229.243081 70.6) (width 0.2) (layer "F.Cu") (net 31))
 (segment (start 182.6864 76.2136) (end 182.6864 79.2944) (width 0.2) (layer "F.Cu") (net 25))
 (segment (start 185.1 74.6) (end 184.3 74.6) (width 0.2) (layer "F.Cu") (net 25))
 (segment (start 184.3 74.6) (end 182.6864 76.2136) (width 0.2) (layer "F.Cu") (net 25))
 (via (at 185.1 74.6) (size 0.6) (drill 0.3) (layers "F.Cu" "B.Cu") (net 25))
 (segment (start 211.1995 73.8995) (end 211.1 73.999) (width 0.2) (layer "B.Cu") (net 25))
 (segment (start 211.72 73.379) (end 211.1995 73.8995) (width 0.2) (layer "B.Cu") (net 25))
 (segment (start 211.1995 73.8995) (end 211.101681 73.997319) (width 0.2) (layer "B.Cu") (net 25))
 (segment (start 185.702681 73.997319) (end 185.1 74.6) (width 0.2) (layer "B.Cu") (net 25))
 (segment (start 211.72 72.059) (end 211.72 73.379) (width 0.2) (layer "B.Cu") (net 25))
 (segment (start 211.101681 73.997319) (end 185.702681 73.997319) (width 0.2) (layer "B.Cu") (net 25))
 (segment (start 177.6 73.2) (end 177.6064 73.2064) (width 0.2) (layer "F.Cu") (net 29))
 (segment (start 177.6064 73.2064) (end 177.6064 79.2944) (width 0.2) (layer "F.Cu") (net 29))
 (via (at 177.6 73.2) (size 0.6) (drill 0.3) (layers "F.Cu" "B.Cu") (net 29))
 (segment (start 178.1 69.4) (end 177.6 69.9) (width 0.2) (layer "B.Cu") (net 29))
 (segment (start 177.6 69.9) (end 177.6 73.2) (width 0.2) (layer "B.Cu") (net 29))
 (segment (start 221.88 72.059) (end 221.88 69.68) (width 0.2) (layer "B.Cu") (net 29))
 (segment (start 221.88 69.68) (end 221.6 69.4) (width 0.2) (layer "B.Cu") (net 29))
 (segment (start 221.6 69.4) (end 178.1 69.4) (width 0.2) (layer "B.Cu") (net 29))
 (segment (start 178.8764 73.7764) (end 178.8764 79.2944) (width 0.2) (layer "F.Cu") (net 28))
 (segment (start 178.8 73.7) (end 178.8764 73.7764) (width 0.2) (layer "F.Cu") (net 28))
 (segment (start 178.8 73.3) (end 178.8 73.7) (width 0.2) (layer "F.Cu") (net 28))
 (via (at 178.8 73.3) (size 0.6) (drill 0.3) (layers "F.Cu" "B.Cu") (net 28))
 (segment (start 178.8 70.2) (end 178.8 73.3) (width 0.2) (layer "B.Cu") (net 28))
 (segment (start 219.34 72.059) (end 219.34 70.14) (width 0.2) (layer "B.Cu") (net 28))
 (segment (start 179.2 69.8) (end 178.8 70.2) (width 0.2) (layer "B.Cu") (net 28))
 (segment (start 219.34 70.14) (end 219 69.8) (width 0.2) (layer "B.Cu") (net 28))
 (segment (start 219 69.8) (end 179.2 69.8) (width 0.2) (layer "B.Cu") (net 28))
 (segment (start 180.1 73.7) (end 180.1464 73.7464) (width 0.2) (layer "F.Cu") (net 27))
 (segment (start 180.1464 73.7464) (end 180.1464 79.2944) (width 0.2) (layer "F.Cu") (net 27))
 (segment (start 180.1 73.4) (end 180.1 73.7) (width 0.2) (layer "F.Cu") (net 27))
 (via (at 180.1 73.4) (size 0.6) (drill 0.3) (layers "F.Cu" "B.Cu") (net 27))
 (segment (start 180.1 70.6) (end 180.1 73.4) (width 0.2) (layer "B.Cu") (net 27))
 (segment (start 216.8 72.059) (end 216.8 70.6) (width 0.2) (layer "B.Cu") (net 27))
 (segment (start 180.5 70.2) (end 180.1 70.6) (width 0.2) (layer "B.Cu") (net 27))
 (segment (start 216.4 70.2) (end 180.5 70.2) (width 0.2) (layer "B.Cu") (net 27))
 (segment (start 216.8 70.6) (end 216.4 70.2) (width 0.2) (layer "B.Cu") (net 27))
 (segment (start 169.9864 69.9136) (end 169.9864 79.2944) (width 0.2) (layer "F.Cu") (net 34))
 (segment (start 237.12 69.72) (end 236.8 69.4) (width 0.2) (layer "F.Cu") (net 34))
 (segment (start 237.12 72.059) (end 237.12 69.72) (width 0.2) (layer "F.Cu") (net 34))
 (segment (start 170.5 69.4) (end 169.9864 69.9136) (width 0.2) (layer "F.Cu") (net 34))
 (segment (start 236.8 69.4) (end 170.5 69.4) (width 0.2) (layer "F.Cu") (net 34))
 (segment (start 226.47 104.8) (end 175.5 104.8) (width 0.2) (layer "F.Cu") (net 7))
 (segment (start 226.96 104.54) (end 226.67 104.83) (width 0.2) (layer "F.Cu") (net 7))
 (segment (start 226.67 104.83) (end 226.5 104.83) (width 0.2) (layer "F.Cu") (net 7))
 (segment (start 175.0664 104.3664) (end 175.0664 96.7944) (width 0.2) (layer "F.Cu") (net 7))
 (segment (start 226.5 104.83) (end 226.47 104.8) (width 0.2) (layer "F.Cu") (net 7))
 (segment (start 226.96 103.3) (end 226.96 104.54) (width 0.2) (layer "F.Cu") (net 7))
 (segment (start 175.5 104.8) (end 175.0664 104.3664) (width 0.2) (layer "F.Cu") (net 7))
 (segment (start 173.7964 104.8964) (end 173.7964 96.7944) (width 0.2) (layer "F.Cu") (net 6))
 (segment (start 229.5 104.93) (end 229.2 105.23) (width 0.2) (layer "F.Cu") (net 6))
 (segment (start 174.13 105.23) (end 173.7964 104.8964) (width 0.2) (layer "F.Cu") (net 6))
 (segment (start 229.5 103.3) (end 229.5 104.93) (width 0.2) (layer "F.Cu") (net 6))
 (segment (start 229.2 105.23) (end 174.13 105.23) (width 0.2) (layer "F.Cu") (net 6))
 (segment (start 184 75.8) (end 183.9564 75.8436) (width 0.2) (layer "F.Cu") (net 24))
 (segment (start 183.9564 75.8436) (end 183.9564 79.2944) (width 0.2) (layer "F.Cu") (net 24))
 (via (at 184 75.8) (size 0.6) (drill 0.3) (layers "F.Cu" "B.Cu") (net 24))
 (segment (start 207.739 73.5) (end 184.7 73.5) (width 0.2) (layer "B.Cu") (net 24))
 (segment (start 184.7 73.5) (end 184 74.2) (width 0.2) (layer "B.Cu") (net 24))
 (segment (start 209.18 72.059) (end 207.739 73.5) (width 0.2) (layer "B.Cu") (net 24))
 (segment (start 184 74.2) (end 184 75.8) (width 0.2) (layer "B.Cu") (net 24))
 (segment (start 237.12 103.3) (end 237.12 106.01) (width 0.2) (layer "F.Cu") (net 3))
 (segment (start 236.7 106.43) (end 170.43 106.43) (width 0.2) (layer "F.Cu") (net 3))
 (segment (start 169.9864 105.9864) (end 169.9864 96.7944) (width 0.2) (layer "F.Cu") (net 3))
 (segment (start 170.43 106.43) (end 169.9864 105.9864) (width 0.2) (layer "F.Cu") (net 3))
 (segment (start 237.12 106.01) (end 236.7 106.43) (width 0.2) (layer "F.Cu") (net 3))
 (segment (start 231.5 105.63) (end 172.83 105.63) (width 0.2) (layer "F.Cu") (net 5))
 (segment (start 232.04 103.3) (end 232.04 105.09) (width 0.2) (layer "F.Cu") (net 5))
 (segment (start 172.5264 105.3264) (end 172.5264 96.7944) (width 0.2) (layer "F.Cu") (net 5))
 (segment (start 172.83 105.63) (end 172.5264 105.3264) (width 0.2) (layer "F.Cu") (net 5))
 (segment (start 232.04 105.09) (end 231.5 105.63) (width 0.2) (layer "F.Cu") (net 5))
 (segment (start 234.58 72.059) (end 234.58 70.08) (width 0.2) (layer "F.Cu") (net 33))
 (segment (start 171.2564 70.2436) (end 171.2564 79.2944) (width 0.2) (layer "F.Cu") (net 33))
 (segment (start 171.7 69.8) (end 171.2564 70.2436) (width 0.2) (layer "F.Cu") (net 33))
 (segment (start 234.3 69.8) (end 171.7 69.8) (width 0.2) (layer "F.Cu") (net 33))
 (segment (start 234.58 70.08) (end 234.3 69.8) (width 0.2) (layer "F.Cu") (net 33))
 (segment (start 239.2 69) (end 169 69) (width 0.2) (layer "F.Cu") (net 35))
 (segment (start 239.66 72.059) (end 239.66 69.46) (width 0.2) (layer "F.Cu") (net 35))
 (segment (start 169 69) (end 168.7164 69.2836) (width 0.2) (layer "F.Cu") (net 35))
 (segment (start 239.66 69.46) (end 239.2 69) (width 0.2) (layer "F.Cu") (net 35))
 (segment (start 168.7164 69.2836) (end 168.7164 79.2944) (width 0.2) (layer "F.Cu") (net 35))
 (segment (start 203.801 73.599) (end 204.1 73.3) (width 0.2) (layer "F.Cu") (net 20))
 (segment (start 204.1 73.3) (end 204.1 72.059) (width 0.2) (layer "F.Cu") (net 20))
 (segment (start 192.9 75.38349) (end 194.684491 73.599) (width 0.2) (layer "F.Cu") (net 20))
 (segment (start 194.684491 73.599) (end 203.801 73.599) (width 0.2) (layer "F.Cu") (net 20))
 (segment (start 192.9 85.7) (end 192.9 75.38349) (width 0.2) (layer "F.Cu") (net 20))
 (segment (start 192.4656 86.1344) (end 192.9 85.7) (width 0.2) (layer "F.Cu") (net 20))
 (segment (start 185.2064 86.1344) (end 192.4656 86.1344) (width 0.2) (layer "F.Cu") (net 20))
 (segment (start 172.5264 70.4736) (end 172.5264 79.2944) (width 0.2) (layer "F.Cu") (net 32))
 (segment (start 231.6 70.2) (end 172.8 70.2) (width 0.2) (layer "F.Cu") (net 32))
 (segment (start 232.04 70.64) (end 231.6 70.2) (width 0.2) (layer "F.Cu") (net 32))
 (segment (start 232.04 72.059) (end 232.04 70.64) (width 0.2) (layer "F.Cu") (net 32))
 (segment (start 172.8 70.2) (end 172.5264 70.4736) (width 0.2) (layer "F.Cu") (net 32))
 (segment (start 176.3364 73.2364) (end 176.3364 79.2944) (width 0.2) (layer "F.Cu") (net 30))
 (segment (start 176.3 73.2) (end 176.3364 73.2364) (width 0.2) (layer "F.Cu") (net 30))
 (via (at 176.3 73.2) (size 0.6) (drill 0.3) (layers "F.Cu" "B.Cu") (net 30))
 (segment (start 176.8 69) (end 176.3 69.5) (width 0.2) (layer "B.Cu") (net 30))
 (segment (start 224.42 72.059) (end 224.42 69.42) (width 0.2) (layer "B.Cu") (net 30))
 (segment (start 224 69) (end 176.8 69) (width 0.2) (layer "B.Cu") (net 30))
 (segment (start 224.42 69.42) (end 224 69) (width 0.2) (layer "B.Cu") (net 30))
 (segment (start 176.3 69.5) (end 176.3 73.2) (width 0.2) (layer "B.Cu") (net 30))
 (segment (start 206.26 101.36) (end 206.64 101.74) (width 0.2) (layer "F.Cu") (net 18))
 (segment (start 194.850176 101.36) (end 206.26 101.36) (width 0.2) (layer "F.Cu") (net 18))
 (segment (start 193.34 99.849824) (end 194.850176 101.36) (width 0.2) (layer "F.Cu") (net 18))
 (segment (start 193.34 88.94) (end 193.34 99.849824) (width 0.2) (layer "F.Cu") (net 18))
 (segment (start 193.0744 88.6744) (end 193.34 88.94) (width 0.2) (layer "F.Cu") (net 18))
 (segment (start 206.64 101.74) (end 206.64 103.3) (width 0.2) (layer "F.Cu") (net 18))
 (segment (start 185.2064 88.6744) (end 193.0744 88.6744) (width 0.2) (layer "F.Cu") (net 18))
 (segment (start 167.83 107.23) (end 167.4464 106.8464) (width 0.2) (layer "F.Cu") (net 1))
 (segment (start 241.8 107.5) (end 241.53 107.23) (width 0.2) (layer "F.Cu") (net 1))
 (segment (start 242.2 107.1) (end 241.8 107.5) (width 0.2) (layer "F.Cu") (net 1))
 (segment (start 241.53 107.23) (end 167.83 107.23) (width 0.2) (layer "F.Cu") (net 1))
 (segment (start 242.2 103.3) (end 242.2 107.1) (width 0.2) (layer "F.Cu") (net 1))
 (segment (start 167.4464 106.8464) (end 167.4464 96.7944) (width 0.2) (layer "F.Cu") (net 1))
 (segment (start 239.66 103.3) (end 239.66 106.17) (width 0.2) (layer "F.Cu") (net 2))
 (segment (start 239 106.83) (end 169.23 106.83) (width 0.2) (layer "F.Cu") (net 2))
 (segment (start 239.66 106.17) (end 239 106.83) (width 0.2) (layer "F.Cu") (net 2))
 (segment (start 169.23 106.83) (end 168.7164 106.3164) (width 0.2) (layer "F.Cu") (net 2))
 (segment (start 168.7164 106.3164) (end 168.7164 96.7944) (width 0.2) (layer "F.Cu") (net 2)))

